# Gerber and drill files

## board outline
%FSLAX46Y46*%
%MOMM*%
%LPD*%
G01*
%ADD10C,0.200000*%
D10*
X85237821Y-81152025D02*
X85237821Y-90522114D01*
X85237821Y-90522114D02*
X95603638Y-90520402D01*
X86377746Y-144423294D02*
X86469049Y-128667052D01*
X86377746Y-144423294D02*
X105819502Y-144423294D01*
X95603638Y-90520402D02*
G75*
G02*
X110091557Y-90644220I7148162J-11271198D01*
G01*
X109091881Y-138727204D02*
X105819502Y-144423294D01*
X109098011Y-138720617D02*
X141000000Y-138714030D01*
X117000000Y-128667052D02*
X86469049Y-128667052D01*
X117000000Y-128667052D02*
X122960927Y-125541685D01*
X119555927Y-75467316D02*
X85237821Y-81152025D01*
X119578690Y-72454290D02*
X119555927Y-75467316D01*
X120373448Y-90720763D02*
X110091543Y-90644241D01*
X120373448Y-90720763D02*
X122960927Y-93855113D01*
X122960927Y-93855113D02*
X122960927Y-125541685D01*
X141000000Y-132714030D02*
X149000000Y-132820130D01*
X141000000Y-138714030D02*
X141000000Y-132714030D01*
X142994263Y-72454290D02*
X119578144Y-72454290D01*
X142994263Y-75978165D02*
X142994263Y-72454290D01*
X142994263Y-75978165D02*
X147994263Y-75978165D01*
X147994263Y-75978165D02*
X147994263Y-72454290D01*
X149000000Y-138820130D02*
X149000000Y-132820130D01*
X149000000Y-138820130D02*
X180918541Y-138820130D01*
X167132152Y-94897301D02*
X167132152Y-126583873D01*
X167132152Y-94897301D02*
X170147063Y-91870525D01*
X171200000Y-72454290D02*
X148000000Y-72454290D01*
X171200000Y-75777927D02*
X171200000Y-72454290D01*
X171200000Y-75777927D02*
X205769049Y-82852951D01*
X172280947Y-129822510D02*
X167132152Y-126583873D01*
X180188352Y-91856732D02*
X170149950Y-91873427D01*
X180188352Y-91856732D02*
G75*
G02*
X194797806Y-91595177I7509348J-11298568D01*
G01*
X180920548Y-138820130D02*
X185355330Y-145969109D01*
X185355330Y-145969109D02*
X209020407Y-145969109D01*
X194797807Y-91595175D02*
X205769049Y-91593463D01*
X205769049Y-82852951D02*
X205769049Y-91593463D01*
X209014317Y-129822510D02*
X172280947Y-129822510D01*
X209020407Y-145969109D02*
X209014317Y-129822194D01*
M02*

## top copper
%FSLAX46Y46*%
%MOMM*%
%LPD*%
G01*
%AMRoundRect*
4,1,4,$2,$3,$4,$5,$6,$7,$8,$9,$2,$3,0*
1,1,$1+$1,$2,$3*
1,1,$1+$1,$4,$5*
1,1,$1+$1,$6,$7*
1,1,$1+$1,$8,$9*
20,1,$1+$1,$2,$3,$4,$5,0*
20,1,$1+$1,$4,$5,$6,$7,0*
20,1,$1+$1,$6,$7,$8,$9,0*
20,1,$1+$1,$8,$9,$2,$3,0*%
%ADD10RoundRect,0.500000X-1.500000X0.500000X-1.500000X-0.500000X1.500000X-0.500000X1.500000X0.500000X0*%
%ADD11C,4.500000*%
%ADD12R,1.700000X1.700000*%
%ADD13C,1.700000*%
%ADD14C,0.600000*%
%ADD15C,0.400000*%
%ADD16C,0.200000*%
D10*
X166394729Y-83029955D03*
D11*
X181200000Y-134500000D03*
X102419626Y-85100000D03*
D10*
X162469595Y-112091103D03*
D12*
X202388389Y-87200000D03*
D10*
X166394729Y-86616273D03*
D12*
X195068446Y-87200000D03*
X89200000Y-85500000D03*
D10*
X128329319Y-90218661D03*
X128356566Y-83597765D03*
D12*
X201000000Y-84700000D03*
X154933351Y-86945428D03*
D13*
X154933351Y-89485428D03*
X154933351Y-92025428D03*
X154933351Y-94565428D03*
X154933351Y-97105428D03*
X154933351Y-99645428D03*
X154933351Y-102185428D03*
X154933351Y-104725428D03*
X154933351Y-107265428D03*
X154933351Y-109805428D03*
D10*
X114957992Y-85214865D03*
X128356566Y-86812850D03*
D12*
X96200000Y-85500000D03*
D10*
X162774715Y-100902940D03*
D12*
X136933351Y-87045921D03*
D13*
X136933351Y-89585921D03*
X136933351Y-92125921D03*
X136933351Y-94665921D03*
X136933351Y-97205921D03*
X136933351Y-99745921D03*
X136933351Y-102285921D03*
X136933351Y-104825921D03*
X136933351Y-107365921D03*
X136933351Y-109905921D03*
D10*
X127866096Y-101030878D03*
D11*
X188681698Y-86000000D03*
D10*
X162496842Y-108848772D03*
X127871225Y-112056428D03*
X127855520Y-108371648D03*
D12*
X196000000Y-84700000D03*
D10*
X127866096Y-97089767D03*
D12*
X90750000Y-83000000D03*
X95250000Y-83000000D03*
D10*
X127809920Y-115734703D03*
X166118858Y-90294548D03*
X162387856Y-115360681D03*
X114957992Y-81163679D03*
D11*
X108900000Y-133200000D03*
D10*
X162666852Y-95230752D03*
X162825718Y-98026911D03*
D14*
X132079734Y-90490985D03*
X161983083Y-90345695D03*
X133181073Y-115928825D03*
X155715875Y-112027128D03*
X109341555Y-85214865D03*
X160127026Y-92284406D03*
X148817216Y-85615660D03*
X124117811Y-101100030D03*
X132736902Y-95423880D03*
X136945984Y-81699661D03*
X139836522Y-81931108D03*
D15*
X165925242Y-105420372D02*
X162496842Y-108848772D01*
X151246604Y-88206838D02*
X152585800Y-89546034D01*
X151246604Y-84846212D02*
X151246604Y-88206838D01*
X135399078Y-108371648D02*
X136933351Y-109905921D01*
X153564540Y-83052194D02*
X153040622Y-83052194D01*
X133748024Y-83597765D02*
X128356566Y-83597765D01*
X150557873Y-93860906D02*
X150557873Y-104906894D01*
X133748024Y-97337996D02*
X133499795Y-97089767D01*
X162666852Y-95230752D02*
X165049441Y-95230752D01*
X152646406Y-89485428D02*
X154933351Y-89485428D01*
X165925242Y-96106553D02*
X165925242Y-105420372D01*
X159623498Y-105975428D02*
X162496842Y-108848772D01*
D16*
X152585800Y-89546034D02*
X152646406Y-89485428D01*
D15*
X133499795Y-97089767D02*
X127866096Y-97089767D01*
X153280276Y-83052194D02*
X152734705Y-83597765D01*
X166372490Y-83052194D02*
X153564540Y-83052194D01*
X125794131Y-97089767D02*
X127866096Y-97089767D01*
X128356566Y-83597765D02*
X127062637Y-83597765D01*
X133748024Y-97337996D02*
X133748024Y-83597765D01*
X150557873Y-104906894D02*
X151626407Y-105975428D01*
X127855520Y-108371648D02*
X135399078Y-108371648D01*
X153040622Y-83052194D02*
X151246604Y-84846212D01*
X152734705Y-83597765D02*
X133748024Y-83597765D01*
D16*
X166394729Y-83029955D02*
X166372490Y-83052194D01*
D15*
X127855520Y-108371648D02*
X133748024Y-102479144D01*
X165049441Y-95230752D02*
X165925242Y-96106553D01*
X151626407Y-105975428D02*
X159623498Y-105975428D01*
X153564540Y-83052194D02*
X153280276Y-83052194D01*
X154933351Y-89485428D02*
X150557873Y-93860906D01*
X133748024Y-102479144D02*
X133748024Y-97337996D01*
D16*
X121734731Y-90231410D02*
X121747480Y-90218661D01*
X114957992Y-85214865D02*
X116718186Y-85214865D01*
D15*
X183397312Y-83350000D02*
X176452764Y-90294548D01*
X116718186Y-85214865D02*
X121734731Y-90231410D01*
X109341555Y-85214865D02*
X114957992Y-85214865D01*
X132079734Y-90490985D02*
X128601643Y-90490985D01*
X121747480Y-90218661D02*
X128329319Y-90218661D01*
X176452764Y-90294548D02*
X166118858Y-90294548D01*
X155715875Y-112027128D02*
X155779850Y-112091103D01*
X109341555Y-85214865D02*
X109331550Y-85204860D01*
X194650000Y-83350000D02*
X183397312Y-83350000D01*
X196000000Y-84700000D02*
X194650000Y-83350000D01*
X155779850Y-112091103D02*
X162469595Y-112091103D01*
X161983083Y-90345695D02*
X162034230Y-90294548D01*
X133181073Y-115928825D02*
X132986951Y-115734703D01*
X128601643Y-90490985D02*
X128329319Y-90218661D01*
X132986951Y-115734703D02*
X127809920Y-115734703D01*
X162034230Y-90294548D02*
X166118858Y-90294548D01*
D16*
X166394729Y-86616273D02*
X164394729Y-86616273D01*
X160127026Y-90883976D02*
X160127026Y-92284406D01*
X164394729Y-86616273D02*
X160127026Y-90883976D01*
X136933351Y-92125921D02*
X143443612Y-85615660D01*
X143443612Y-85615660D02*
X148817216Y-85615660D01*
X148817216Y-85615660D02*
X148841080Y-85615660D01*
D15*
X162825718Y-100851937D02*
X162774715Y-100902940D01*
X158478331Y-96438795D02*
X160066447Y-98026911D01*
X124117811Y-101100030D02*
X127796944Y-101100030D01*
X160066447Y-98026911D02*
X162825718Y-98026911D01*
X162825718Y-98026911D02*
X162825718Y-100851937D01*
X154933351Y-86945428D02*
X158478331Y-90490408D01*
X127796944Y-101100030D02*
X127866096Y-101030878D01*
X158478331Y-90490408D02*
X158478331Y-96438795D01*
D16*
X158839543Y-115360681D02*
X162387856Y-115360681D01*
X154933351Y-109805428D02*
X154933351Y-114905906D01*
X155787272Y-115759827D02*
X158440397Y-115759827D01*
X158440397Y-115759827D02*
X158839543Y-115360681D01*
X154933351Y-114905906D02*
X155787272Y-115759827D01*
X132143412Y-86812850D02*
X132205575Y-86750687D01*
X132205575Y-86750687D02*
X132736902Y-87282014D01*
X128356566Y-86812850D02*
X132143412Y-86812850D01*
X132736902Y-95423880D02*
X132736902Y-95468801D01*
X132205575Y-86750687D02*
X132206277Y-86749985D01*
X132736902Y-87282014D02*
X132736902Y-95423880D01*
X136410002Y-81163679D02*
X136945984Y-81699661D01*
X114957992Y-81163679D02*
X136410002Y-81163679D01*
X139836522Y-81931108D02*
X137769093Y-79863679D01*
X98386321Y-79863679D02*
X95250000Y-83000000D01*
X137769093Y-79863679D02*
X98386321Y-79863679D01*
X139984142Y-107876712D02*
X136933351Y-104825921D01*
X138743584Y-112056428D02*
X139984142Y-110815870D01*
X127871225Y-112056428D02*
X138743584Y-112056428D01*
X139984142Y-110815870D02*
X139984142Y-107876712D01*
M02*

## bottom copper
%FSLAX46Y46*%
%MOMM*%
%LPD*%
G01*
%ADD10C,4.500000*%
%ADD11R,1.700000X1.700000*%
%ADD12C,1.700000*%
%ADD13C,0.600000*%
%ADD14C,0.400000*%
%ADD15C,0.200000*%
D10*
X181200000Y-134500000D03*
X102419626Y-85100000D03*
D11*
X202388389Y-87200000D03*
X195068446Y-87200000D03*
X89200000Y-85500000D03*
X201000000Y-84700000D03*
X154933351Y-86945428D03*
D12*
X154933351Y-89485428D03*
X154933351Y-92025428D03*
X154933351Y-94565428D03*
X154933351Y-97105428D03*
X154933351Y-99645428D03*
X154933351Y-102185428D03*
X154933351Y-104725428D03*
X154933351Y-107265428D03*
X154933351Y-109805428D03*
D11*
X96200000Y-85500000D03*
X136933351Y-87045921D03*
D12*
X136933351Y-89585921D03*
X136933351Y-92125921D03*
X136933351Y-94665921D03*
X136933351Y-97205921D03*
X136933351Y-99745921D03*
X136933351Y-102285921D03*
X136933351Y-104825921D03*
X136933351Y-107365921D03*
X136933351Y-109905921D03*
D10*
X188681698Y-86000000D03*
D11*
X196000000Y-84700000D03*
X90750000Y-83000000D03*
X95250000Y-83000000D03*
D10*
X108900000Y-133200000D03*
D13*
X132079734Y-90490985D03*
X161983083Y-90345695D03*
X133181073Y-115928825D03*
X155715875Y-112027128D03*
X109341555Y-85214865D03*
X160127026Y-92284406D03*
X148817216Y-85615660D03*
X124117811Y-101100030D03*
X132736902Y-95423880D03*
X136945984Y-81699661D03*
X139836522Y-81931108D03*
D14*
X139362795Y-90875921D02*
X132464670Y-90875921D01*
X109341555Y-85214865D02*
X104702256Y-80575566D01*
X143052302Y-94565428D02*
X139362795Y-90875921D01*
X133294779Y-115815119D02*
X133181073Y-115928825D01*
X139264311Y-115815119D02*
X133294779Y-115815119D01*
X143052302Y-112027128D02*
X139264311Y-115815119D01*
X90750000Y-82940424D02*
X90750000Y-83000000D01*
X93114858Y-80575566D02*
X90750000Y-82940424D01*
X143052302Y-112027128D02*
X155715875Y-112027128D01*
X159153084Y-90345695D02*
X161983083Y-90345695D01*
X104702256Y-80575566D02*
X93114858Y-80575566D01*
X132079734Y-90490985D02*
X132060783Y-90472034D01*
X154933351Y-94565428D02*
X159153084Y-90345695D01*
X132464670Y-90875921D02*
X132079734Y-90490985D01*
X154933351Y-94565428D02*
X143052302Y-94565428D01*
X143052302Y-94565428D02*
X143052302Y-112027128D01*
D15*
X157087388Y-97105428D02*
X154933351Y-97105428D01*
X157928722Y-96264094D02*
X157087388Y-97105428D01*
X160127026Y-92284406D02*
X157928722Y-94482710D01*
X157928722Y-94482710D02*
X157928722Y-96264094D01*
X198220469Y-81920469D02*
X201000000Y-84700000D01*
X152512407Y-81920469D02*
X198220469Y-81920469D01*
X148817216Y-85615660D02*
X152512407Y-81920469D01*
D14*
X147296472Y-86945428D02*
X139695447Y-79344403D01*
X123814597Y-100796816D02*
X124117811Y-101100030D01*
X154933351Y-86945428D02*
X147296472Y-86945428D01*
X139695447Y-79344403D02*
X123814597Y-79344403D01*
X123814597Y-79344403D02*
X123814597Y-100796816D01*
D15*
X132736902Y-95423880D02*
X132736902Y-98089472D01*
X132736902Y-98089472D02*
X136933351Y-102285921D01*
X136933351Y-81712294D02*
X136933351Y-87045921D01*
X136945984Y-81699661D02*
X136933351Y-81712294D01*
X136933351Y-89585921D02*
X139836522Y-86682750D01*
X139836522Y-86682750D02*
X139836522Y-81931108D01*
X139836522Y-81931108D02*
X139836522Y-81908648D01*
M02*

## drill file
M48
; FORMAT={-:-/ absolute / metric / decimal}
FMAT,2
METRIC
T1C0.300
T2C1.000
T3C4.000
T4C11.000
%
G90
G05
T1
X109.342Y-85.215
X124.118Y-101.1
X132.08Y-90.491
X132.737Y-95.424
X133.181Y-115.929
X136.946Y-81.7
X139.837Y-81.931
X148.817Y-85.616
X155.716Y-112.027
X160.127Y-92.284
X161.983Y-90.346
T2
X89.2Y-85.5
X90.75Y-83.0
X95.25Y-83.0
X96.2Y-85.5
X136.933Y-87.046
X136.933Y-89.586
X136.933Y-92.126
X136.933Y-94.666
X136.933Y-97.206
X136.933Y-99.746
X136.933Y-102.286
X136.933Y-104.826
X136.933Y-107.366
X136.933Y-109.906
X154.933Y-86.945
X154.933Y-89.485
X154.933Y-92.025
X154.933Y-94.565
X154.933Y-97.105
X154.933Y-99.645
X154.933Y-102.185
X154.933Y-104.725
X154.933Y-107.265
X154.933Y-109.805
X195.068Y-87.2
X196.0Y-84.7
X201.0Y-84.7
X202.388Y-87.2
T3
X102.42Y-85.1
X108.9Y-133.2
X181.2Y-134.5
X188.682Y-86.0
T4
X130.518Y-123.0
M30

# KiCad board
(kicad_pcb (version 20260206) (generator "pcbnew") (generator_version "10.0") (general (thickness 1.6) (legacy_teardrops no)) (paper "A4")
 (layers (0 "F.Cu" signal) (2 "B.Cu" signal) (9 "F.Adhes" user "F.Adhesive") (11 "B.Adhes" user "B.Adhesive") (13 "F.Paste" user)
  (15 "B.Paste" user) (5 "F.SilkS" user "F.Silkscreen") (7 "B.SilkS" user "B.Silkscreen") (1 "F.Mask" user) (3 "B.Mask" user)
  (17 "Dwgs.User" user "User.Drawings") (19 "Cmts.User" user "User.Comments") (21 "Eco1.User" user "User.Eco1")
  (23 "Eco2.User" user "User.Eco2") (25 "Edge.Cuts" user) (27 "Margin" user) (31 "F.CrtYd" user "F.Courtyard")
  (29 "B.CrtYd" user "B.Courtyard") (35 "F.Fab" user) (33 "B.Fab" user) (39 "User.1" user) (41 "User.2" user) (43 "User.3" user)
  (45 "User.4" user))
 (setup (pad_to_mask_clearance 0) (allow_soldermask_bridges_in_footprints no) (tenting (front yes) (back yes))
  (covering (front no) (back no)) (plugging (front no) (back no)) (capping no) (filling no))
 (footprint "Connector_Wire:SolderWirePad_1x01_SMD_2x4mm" (layer "F.Cu") (at 166.394729 83.029955 -90)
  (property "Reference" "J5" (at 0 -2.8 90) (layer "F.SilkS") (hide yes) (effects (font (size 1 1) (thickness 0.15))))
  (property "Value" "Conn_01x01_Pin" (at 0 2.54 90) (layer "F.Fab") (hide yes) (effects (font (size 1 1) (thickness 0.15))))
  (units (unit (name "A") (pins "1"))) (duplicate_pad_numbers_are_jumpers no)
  (pad "1" smd roundrect (at 0 0 270) (size 2 4) (layers "F.Cu" "F.Mask") (roundrect_rratio 0.25) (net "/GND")))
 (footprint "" (layer "F.Cu") (at 199.537516 63.787243)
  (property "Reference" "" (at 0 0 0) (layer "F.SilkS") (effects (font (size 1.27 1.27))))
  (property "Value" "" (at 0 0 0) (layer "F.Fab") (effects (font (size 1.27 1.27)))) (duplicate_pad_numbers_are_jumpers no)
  (pad "" np_thru_hole circle (at -18.337516 70.712757) (size 4.5 4.5) (drill 4) (layers "*.Cu" "*.Mask")))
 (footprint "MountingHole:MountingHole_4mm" (layer "F.Cu") (at 102.419626 85.1)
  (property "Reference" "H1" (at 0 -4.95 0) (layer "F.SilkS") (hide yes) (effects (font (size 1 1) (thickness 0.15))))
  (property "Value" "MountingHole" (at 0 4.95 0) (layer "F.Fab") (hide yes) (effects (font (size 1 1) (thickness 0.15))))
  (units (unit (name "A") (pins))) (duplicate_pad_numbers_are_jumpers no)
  (pad "" np_thru_hole circle (at 0 0) (size 4.5 4.5) (drill 4) (layers "*.Cu" "*.Mask")))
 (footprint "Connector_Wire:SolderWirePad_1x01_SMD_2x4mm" (layer "F.Cu") (at 162.469595 112.091103 -90)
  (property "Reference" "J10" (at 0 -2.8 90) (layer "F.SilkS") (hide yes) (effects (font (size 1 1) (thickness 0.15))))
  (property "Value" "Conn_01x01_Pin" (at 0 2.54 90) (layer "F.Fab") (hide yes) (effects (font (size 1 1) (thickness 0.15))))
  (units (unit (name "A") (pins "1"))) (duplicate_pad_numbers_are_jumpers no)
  (pad "1" smd roundrect (at 0 0 270) (size 2 4) (layers "F.Cu" "F.Mask") (roundrect_rratio 0.25) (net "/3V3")))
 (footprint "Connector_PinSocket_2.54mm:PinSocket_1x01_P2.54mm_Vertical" (layer "F.Cu") (at 202.388389 87.2)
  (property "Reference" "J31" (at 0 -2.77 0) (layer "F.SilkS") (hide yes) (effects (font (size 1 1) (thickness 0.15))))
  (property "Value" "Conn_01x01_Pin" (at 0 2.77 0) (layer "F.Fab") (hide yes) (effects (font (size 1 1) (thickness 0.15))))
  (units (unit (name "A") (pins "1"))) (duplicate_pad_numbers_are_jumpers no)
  (pad "1" thru_hole rect (at 0 0) (size 1.7 1.7) (drill 1) (layers "*.Cu" "*.Mask") (remove_unused_layers no)
   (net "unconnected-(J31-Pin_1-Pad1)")))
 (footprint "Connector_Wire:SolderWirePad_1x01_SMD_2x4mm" (layer "F.Cu") (at 166.394729 86.616273 -90)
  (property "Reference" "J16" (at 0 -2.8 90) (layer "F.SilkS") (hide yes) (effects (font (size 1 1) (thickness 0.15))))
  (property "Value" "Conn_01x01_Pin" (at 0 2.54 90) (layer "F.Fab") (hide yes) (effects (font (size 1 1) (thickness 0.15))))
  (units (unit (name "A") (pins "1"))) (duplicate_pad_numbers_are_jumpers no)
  (pad "1" smd roundrect (at 0 0 270) (size 2 4) (layers "F.Cu" "F.Mask") (roundrect_rratio 0.25) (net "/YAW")))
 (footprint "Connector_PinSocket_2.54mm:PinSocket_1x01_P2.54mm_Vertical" (layer "F.Cu") (at 195.068446 87.2)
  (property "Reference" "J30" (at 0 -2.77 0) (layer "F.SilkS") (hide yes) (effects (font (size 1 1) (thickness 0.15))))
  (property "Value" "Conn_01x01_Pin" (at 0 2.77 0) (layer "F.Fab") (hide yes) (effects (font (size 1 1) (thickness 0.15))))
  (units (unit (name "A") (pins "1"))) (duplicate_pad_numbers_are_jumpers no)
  (pad "1" thru_hole rect (at 0 0) (size 1.7 1.7) (drill 1) (layers "*.Cu" "*.Mask") (remove_unused_layers no)
   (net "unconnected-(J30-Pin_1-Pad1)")))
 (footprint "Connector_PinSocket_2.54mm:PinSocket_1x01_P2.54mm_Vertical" (layer "F.Cu") (at 89.2 85.5)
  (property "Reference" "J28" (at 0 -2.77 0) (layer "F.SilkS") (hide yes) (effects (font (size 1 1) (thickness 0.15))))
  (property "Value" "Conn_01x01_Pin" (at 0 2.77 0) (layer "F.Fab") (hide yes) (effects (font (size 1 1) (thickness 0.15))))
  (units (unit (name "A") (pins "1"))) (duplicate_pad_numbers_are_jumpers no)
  (pad "1" thru_hole rect (at 0 0) (size 1.7 1.7) (drill 1) (layers "*.Cu" "*.Mask") (remove_unused_layers no)
   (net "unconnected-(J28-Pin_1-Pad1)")))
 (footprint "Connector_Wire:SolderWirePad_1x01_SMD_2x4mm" (layer "F.Cu") (at 128.329319 90.218661 -90)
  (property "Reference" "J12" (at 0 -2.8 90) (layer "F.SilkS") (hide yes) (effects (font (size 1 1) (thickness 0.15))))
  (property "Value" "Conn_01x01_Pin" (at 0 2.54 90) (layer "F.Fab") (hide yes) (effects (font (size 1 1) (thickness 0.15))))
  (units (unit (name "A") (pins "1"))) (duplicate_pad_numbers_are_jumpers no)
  (pad "1" smd roundrect (at 0 0 270) (size 2 4) (layers "F.Cu" "F.Mask") (roundrect_rratio 0.25) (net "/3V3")))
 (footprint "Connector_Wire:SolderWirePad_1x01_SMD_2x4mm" (layer "F.Cu") (at 128.356566 83.597765 -90)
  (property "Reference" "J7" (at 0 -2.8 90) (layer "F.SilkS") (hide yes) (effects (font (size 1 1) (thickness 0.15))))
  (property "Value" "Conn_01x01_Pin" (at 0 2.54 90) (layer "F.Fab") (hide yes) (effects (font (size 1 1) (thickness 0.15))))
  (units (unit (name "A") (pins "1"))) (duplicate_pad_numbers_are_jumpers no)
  (pad "1" smd roundrect (at 0 0 270) (size 2 4) (layers "F.Cu" "F.Mask") (roundrect_rratio 0.25) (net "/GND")))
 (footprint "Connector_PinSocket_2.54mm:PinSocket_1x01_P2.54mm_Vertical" (layer "F.Cu") (at 201 84.7)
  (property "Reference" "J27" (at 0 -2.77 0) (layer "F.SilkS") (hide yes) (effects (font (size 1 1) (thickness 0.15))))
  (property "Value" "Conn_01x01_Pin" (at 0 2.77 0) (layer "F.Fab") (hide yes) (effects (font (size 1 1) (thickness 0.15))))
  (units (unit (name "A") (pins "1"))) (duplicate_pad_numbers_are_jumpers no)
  (pad "1" thru_hole rect (at 0 0) (size 1.7 1.7) (drill 1) (layers "*.Cu" "*.Mask") (remove_unused_layers no) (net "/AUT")))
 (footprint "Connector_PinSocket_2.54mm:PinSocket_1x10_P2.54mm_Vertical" (layer "F.Cu") (at 154.933351 86.945428)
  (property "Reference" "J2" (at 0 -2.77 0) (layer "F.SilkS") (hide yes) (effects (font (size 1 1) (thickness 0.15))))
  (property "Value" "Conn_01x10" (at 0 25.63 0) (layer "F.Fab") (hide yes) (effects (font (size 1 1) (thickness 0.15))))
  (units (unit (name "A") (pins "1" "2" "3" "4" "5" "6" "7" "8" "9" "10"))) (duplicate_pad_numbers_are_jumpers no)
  (pad "1" thru_hole rect (at 0 0) (size 1.7 1.7) (drill 1) (layers "*.Cu" "*.Mask") (remove_unused_layers no) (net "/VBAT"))
  (pad "2" thru_hole circle (at 0 2.54) (size 1.7 1.7) (drill 1) (layers "*.Cu" "*.Mask") (remove_unused_layers no) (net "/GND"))
  (pad "3" thru_hole circle (at 0 5.08) (size 1.7 1.7) (drill 1) (layers "*.Cu" "*.Mask") (remove_unused_layers no) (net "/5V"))
  (pad "4" thru_hole circle (at 0 7.62) (size 1.7 1.7) (drill 1) (layers "*.Cu" "*.Mask") (remove_unused_layers no) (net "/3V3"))
  (pad "5" thru_hole circle (at 0 10.16) (size 1.7 1.7) (drill 1) (layers "*.Cu" "*.Mask") (remove_unused_layers no) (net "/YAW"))
  (pad "6" thru_hole circle (at 0 12.7) (size 1.7 1.7) (drill 1) (layers "*.Cu" "*.Mask") (remove_unused_layers no)
   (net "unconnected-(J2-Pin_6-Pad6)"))
  (pad "7" thru_hole circle (at 0 15.24) (size 1.7 1.7) (drill 1) (layers "*.Cu" "*.Mask") (remove_unused_layers no)
   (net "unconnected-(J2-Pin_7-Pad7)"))
  (pad "8" thru_hole circle (at 0 17.78) (size 1.7 1.7) (drill 1) (layers "*.Cu" "*.Mask") (remove_unused_layers no)
   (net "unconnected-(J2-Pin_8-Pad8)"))
  (pad "9" thru_hole circle (at 0 20.32) (size 1.7 1.7) (drill 1) (layers "*.Cu" "*.Mask") (remove_unused_layers no)
   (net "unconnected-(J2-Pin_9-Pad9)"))
  (pad "10" thru_hole circle (at 0 22.86) (size 1.7 1.7) (drill 1) (layers "*.Cu" "*.Mask") (remove_unused_layers no) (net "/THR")))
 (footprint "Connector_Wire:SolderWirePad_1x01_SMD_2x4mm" (layer "F.Cu") (at 114.957992 85.214865 -90)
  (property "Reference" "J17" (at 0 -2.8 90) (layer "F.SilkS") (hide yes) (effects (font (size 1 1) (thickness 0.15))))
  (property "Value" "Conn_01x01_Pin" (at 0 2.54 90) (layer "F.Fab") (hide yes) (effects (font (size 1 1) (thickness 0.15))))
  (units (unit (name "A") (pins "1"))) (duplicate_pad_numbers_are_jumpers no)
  (pad "1" smd roundrect (at 0 0 270) (size 2 4) (layers "F.Cu" "F.Mask") (roundrect_rratio 0.25) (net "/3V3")))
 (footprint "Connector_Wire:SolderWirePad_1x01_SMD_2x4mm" (layer "F.Cu") (at 128.356566 86.81285 -90)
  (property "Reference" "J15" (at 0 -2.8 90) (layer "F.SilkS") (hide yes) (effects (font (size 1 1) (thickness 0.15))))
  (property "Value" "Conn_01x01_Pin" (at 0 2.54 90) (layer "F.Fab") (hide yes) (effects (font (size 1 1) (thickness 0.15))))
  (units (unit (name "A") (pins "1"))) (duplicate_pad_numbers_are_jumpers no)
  (pad "1" smd roundrect (at 0 0 270) (size 2 4) (layers "F.Cu" "F.Mask") (roundrect_rratio 0.25) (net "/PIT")))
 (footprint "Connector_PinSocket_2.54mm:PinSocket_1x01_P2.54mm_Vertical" (layer "F.Cu") (at 96.2 85.5)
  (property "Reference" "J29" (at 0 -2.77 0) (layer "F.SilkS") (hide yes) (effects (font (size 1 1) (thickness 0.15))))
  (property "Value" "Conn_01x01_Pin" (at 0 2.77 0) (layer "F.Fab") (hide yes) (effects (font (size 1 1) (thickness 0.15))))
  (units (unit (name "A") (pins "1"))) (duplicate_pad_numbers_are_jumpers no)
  (pad "1" thru_hole rect (at 0 0) (size 1.7 1.7) (drill 1) (layers "*.Cu" "*.Mask") (remove_unused_layers no)
   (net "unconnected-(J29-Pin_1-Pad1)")))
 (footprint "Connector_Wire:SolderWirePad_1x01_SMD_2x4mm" (layer "F.Cu") (at 162.774715 100.90294 -90)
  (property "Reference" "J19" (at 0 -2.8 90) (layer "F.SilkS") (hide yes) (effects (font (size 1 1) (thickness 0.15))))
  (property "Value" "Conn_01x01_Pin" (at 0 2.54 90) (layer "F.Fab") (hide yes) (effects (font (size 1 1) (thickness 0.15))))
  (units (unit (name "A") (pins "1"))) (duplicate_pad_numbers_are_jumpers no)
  (pad "1" smd roundrect (at 0 0 270) (size 2 4) (layers "F.Cu" "F.Mask") (roundrect_rratio 0.25) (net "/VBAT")))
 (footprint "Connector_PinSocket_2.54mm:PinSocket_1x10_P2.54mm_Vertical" (layer "F.Cu") (at 136.933351 87.045921)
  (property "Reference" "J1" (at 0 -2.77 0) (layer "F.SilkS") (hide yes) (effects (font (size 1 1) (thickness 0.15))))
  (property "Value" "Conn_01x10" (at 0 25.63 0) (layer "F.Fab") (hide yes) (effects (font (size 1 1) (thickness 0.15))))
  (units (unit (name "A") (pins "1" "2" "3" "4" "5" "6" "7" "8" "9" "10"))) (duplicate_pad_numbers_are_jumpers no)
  (pad "1" thru_hole rect (at 0 0) (size 1.7 1.7) (drill 1) (layers "*.Cu" "*.Mask") (remove_unused_layers no) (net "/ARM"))
  (pad "2" thru_hole circle (at 0 2.54) (size 1.7 1.7) (drill 1) (layers "*.Cu" "*.Mask") (remove_unused_layers no) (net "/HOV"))
  (pad "3" thru_hole circle (at 0 5.08) (size 1.7 1.7) (drill 1) (layers "*.Cu" "*.Mask") (remove_unused_layers no) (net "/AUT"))
  (pad "4" thru_hole circle (at 0 7.62) (size 1.7 1.7) (drill 1) (layers "*.Cu" "*.Mask") (remove_unused_layers no) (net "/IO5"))
  (pad "5" thru_hole circle (at 0 10.16) (size 1.7 1.7) (drill 1) (layers "*.Cu" "*.Mask") (remove_unused_layers no) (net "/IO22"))
  (pad "6" thru_hole circle (at 0 12.7) (size 1.7 1.7) (drill 1) (layers "*.Cu" "*.Mask") (remove_unused_layers no) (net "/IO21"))
  (pad "7" thru_hole circle (at 0 15.24) (size 1.7 1.7) (drill 1) (layers "*.Cu" "*.Mask") (remove_unused_layers no) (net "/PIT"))
  (pad "8" thru_hole circle (at 0 17.78) (size 1.7 1.7) (drill 1) (layers "*.Cu" "*.Mask") (remove_unused_layers no) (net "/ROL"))
  (pad "9" thru_hole circle (at 0 20.32) (size 1.7 1.7) (drill 1) (layers "*.Cu" "*.Mask") (remove_unused_layers no) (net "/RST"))
  (pad "10" thru_hole circle (at 0 22.86) (size 1.7 1.7) (drill 1) (layers "*.Cu" "*.Mask") (remove_unused_layers no) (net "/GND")))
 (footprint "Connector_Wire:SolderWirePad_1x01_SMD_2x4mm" (layer "F.Cu") (at 127.866096 101.030878 -90)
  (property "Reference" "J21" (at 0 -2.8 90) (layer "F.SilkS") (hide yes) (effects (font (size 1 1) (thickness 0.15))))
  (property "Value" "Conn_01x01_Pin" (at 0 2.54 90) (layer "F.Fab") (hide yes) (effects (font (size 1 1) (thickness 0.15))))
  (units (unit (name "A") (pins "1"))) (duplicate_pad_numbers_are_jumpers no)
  (pad "1" smd roundrect (at 0 0 270) (size 2 4) (layers "F.Cu" "F.Mask") (roundrect_rratio 0.25) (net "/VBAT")))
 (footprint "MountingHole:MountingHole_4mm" (layer "F.Cu") (at 188.681698 86)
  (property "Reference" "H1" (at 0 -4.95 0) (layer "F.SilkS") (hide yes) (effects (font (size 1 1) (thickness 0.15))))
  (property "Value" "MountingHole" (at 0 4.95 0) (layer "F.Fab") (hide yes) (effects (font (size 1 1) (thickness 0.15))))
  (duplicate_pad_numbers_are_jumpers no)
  (pad "" np_thru_hole circle (at 0 0) (size 4.5 4.5) (drill 4) (layers "*.Cu" "*.Mask")))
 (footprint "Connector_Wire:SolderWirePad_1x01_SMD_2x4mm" (layer "F.Cu") (at 162.496842 108.848772 -90)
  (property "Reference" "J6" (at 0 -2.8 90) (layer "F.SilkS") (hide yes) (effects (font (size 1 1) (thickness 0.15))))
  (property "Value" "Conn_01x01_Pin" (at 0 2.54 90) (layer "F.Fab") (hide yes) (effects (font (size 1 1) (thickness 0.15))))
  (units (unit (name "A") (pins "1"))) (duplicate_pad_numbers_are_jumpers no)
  (pad "1" smd roundrect (at 0 0 270) (size 2 4) (layers "F.Cu" "F.Mask") (roundrect_rratio 0.25) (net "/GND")))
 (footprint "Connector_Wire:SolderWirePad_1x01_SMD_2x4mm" (layer "F.Cu") (at 127.871225 112.056428 -90)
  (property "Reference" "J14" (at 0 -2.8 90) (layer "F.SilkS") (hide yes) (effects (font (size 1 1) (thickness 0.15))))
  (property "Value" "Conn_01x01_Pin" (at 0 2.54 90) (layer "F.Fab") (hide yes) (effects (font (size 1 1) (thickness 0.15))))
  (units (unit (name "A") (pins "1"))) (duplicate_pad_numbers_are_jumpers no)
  (pad "1" smd roundrect (at 0 0 270) (size 2 4) (layers "F.Cu" "F.Mask") (roundrect_rratio 0.25) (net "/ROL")))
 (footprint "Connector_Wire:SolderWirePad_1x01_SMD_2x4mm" (layer "F.Cu") (at 127.85552 108.371648 -90)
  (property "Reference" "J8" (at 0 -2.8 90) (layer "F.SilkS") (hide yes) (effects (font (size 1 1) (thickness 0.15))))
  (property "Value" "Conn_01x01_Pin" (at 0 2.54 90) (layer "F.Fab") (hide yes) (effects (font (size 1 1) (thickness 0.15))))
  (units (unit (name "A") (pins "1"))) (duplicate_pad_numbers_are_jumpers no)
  (pad "1" smd roundrect (at 0 0 270) (size 2 4) (layers "F.Cu" "F.Mask") (roundrect_rratio 0.25) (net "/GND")))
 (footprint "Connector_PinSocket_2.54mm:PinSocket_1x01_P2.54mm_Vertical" (layer "F.Cu") (at 196 84.7)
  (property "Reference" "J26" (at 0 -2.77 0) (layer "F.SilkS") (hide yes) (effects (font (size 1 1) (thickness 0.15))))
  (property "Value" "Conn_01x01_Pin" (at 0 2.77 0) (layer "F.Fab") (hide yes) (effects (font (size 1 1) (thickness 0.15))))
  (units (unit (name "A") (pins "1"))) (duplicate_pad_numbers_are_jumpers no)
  (pad "1" thru_hole rect (at 0 0) (size 1.7 1.7) (drill 1) (layers "*.Cu" "*.Mask") (remove_unused_layers no) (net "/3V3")))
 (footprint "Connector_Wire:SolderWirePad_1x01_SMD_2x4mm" (layer "F.Cu") (at 127.866096 97.089767 -90)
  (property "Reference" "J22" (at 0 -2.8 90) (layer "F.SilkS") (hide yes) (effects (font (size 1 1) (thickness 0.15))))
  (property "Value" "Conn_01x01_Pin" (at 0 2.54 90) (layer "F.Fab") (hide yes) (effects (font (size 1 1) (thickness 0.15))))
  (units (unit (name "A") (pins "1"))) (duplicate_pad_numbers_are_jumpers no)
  (pad "1" smd roundrect (at 0 0 270) (size 2 4) (layers "F.Cu" "F.Mask") (roundrect_rratio 0.25) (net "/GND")))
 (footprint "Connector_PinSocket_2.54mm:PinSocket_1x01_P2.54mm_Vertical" (layer "F.Cu") (at 90.75 83)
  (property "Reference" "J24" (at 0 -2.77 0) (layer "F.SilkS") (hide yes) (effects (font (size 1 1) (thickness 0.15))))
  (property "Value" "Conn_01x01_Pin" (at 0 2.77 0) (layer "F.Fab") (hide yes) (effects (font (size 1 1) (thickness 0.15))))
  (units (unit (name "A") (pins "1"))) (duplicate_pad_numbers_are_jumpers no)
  (pad "1" thru_hole rect (at 0 0) (size 1.7 1.7) (drill 1) (layers "*.Cu" "*.Mask") (remove_unused_layers no) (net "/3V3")))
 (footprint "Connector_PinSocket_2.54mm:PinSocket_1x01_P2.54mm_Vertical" (layer "F.Cu") (at 95.25 83)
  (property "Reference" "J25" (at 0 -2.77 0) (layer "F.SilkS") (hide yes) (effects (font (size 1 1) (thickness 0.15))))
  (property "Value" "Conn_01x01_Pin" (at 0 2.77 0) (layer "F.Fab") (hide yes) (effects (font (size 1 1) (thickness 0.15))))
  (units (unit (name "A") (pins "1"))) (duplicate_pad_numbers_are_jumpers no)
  (pad "1" thru_hole rect (at 0 0) (size 1.7 1.7) (drill 1) (layers "*.Cu" "*.Mask") (remove_unused_layers no) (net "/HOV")))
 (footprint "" (layer "F.Cu") (at 131 123 180)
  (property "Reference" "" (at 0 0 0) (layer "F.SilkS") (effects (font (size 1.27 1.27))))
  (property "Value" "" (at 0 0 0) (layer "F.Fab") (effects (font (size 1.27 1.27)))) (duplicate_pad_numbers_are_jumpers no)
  (pad "" np_thru_hole circle (at 0.482324 0 180) (size 11 11) (drill 11) (layers "*.Cu" "*.Mask")))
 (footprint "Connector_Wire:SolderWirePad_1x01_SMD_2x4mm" (layer "F.Cu") (at 127.80992 115.734703 -90)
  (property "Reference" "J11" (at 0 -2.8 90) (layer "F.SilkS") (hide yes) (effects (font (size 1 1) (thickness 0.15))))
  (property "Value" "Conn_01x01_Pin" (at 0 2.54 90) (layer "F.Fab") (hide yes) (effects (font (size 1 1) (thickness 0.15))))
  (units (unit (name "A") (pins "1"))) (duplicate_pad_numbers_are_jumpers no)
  (pad "1" smd roundrect (at 0 0 270) (size 2 4) (layers "F.Cu" "F.Mask") (roundrect_rratio 0.25) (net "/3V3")))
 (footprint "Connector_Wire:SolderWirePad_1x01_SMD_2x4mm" (layer "F.Cu") (at 166.118858 90.294548 -90)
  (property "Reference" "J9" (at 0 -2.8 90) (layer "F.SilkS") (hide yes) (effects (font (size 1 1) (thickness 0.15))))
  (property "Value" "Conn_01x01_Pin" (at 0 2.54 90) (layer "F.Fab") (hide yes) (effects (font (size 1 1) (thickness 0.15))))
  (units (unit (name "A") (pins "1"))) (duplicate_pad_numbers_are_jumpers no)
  (pad "1" smd roundrect (at 0 0 270) (size 2 4) (layers "F.Cu" "F.Mask") (roundrect_rratio 0.25) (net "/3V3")))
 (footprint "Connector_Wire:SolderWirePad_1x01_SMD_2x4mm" (layer "F.Cu") (at 162.387856 115.360681 -90)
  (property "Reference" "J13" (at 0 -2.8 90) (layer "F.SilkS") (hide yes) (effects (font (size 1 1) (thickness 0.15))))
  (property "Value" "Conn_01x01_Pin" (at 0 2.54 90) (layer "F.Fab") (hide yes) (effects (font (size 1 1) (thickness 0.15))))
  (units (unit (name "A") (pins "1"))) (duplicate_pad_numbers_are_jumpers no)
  (pad "1" smd roundrect (at 0 0 270) (size 2 4) (layers "F.Cu" "F.Mask") (roundrect_rratio 0.25) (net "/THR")))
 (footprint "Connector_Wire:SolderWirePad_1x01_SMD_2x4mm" (layer "F.Cu") (at 114.957992 81.163679 -90)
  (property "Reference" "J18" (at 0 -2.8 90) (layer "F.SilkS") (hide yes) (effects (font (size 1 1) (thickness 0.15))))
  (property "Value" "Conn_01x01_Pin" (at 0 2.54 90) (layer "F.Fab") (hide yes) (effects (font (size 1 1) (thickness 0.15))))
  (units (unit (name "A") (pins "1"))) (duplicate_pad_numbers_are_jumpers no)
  (pad "1" smd roundrect (at 0 0 270) (size 2 4) (layers "F.Cu" "F.Mask") (roundrect_rratio 0.25) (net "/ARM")))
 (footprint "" (layer "F.Cu") (at 98.892008 62.425329)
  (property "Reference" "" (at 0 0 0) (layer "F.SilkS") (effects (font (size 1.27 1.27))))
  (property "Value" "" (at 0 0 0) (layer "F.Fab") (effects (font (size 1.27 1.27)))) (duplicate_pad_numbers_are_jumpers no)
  (pad "" np_thru_hole circle (at 10.007992 70.774671) (size 4.5 4.5) (drill 4) (layers "*.Cu" "*.Mask")))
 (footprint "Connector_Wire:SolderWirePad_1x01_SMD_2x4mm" (layer "F.Cu") (at 162.666852 95.230752 -90)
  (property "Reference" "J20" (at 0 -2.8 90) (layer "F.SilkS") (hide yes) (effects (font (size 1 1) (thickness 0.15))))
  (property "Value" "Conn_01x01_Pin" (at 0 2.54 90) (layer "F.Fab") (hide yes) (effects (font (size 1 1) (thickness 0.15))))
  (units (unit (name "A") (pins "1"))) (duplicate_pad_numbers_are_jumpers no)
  (pad "1" smd roundrect (at 0 0 270) (size 2 4) (layers "F.Cu" "F.Mask") (roundrect_rratio 0.25) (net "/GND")))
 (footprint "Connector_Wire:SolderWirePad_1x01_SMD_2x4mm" (layer "F.Cu") (at 162.825718 98.026911 -90)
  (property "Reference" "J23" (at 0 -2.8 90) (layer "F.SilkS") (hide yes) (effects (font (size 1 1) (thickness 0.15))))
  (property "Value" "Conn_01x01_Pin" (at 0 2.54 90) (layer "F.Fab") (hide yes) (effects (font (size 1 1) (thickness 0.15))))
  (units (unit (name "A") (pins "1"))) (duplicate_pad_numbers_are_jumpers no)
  (pad "1" smd roundrect (at 0 0 270) (size 2 4) (layers "F.Cu" "F.Mask") (roundrect_rratio 0.25) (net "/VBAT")))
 (gr_line (start 85.237821 81.152025) (end 85.237821 90.522114) (stroke (width 0.2) (type solid)) (layer "Edge.Cuts"))
 (gr_line (start 85.237821 90.522114) (end 95.603638 90.520402) (stroke (width 0.2) (type solid)) (layer "Edge.Cuts"))
 (gr_line (start 86.377746 144.423294) (end 86.469049 128.667052) (stroke (width 0.2) (type solid)) (layer "Edge.Cuts"))
 (gr_line (start 86.377746 144.423294) (end 105.819502 144.423294) (stroke (width 0.2) (type solid)) (layer "Edge.Cuts"))
 (gr_arc (start 95.603638 90.520402) (mid 102.865857 88.445339) (end 110.091543 90.644241) (stroke (width 0.2) (type solid))
  (layer "Edge.Cuts"))
 (gr_line (start 109.091881 138.727204) (end 105.819502 144.423294) (stroke (width 0.2) (type solid)) (layer "Edge.Cuts"))
 (gr_line (start 109.098011 138.720617) (end 141 138.71403) (stroke (width 0.2) (type solid)) (layer "Edge.Cuts"))
 (gr_line (start 117 128.667052) (end 86.469049 128.667052) (stroke (width 0.2) (type solid)) (layer "Edge.Cuts"))
 (gr_line (start 117 128.667052) (end 122.960927 125.541685) (stroke (width 0.2) (type solid)) (layer "Edge.Cuts"))
 (gr_line (start 119.555927 75.467316) (end 85.237821 81.152025) (stroke (width 0.2) (type solid)) (layer "Edge.Cuts"))
 (gr_line (start 119.57869 72.45429) (end 119.555927 75.467316) (stroke (width 0.2) (type solid)) (layer "Edge.Cuts"))
 (gr_line (start 120.373448 90.720763) (end 110.091543 90.644241) (stroke (width 0.2) (type solid)) (layer "Edge.Cuts"))
 (gr_line (start 120.373448 90.720763) (end 122.960927 93.855113) (stroke (width 0.2) (type solid)) (layer "Edge.Cuts"))
 (gr_line (start 122.960927 93.855113) (end 122.960927 125.541685) (stroke (width 0.2) (type solid)) (layer "Edge.Cuts"))
 (gr_line (start 141 132.71403) (end 149 132.82013) (stroke (width 0.2) (type solid)) (layer "Edge.Cuts"))
 (gr_line (start 141 138.71403) (end 141 132.71403) (stroke (width 0.2) (type solid)) (layer "Edge.Cuts"))
 (gr_line (start 142.994263 72.45429) (end 119.578144 72.45429) (stroke (width 0.2) (type solid)) (layer "Edge.Cuts"))
 (gr_line (start 142.994263 75.978165) (end 142.994263 72.45429) (stroke (width 0.2) (type solid)) (layer "Edge.Cuts"))
 (gr_line (start 142.994263 75.978165) (end 147.994263 75.978165) (stroke (width 0.2) (type solid)) (layer "Edge.Cuts"))
 (gr_line (start 147.994263 75.978165) (end 147.994263 72.45429) (stroke (width 0.2) (type solid)) (layer "Edge.Cuts"))
 (gr_line (start 149 138.82013) (end 149 132.82013) (stroke (width 0.2) (type solid)) (layer "Edge.Cuts"))
 (gr_line (start 149 138.82013) (end 180.918541 138.82013) (stroke (width 0.2) (type solid)) (layer "Edge.Cuts"))
 (gr_line (start 167.132152 94.897301) (end 167.132152 126.583873) (stroke (width 0.2) (type solid)) (layer "Edge.Cuts"))
 (gr_line (start 167.132152 94.897301) (end 170.147063 91.870525) (stroke (width 0.2) (type solid)) (layer "Edge.Cuts"))
 (gr_line (start 171.2 72.45429) (end 148 72.45429) (stroke (width 0.2) (type solid)) (layer "Edge.Cuts"))
 (gr_line (start 171.2 75.777927) (end 171.2 72.45429) (stroke (width 0.2) (type solid)) (layer "Edge.Cuts"))
 (gr_line (start 171.2 75.777927) (end 205.769049 82.852951) (stroke (width 0.2) (type solid)) (layer "Edge.Cuts"))
 (gr_line (start 172.280947 129.82251) (end 167.132152 126.583873) (stroke (width 0.2) (type solid)) (layer "Edge.Cuts"))
 (gr_line (start 180.188352 91.856732) (end 170.14995 91.873427) (stroke (width 0.2) (type solid)) (layer "Edge.Cuts"))
 (gr_arc (start 180.188352 91.856732) (mid 187.454858 89.591048) (end 194.797807 91.595176) (stroke (width 0.2) (type solid))
  (layer "Edge.Cuts"))
 (gr_line (start 180.920548 138.82013) (end 185.35533 145.969109) (stroke (width 0.2) (type solid)) (layer "Edge.Cuts"))
 (gr_line (start 185.35533 145.969109) (end 209.020407 145.969109) (stroke (width 0.2) (type solid)) (layer "Edge.Cuts"))
 (gr_line (start 194.797807 91.595175) (end 205.769049 91.593463) (stroke (width 0.2) (type solid)) (layer "Edge.Cuts"))
 (gr_line (start 205.769049 82.852951) (end 205.769049 91.593463) (stroke (width 0.2) (type solid)) (layer "Edge.Cuts"))
 (gr_line (start 209.014317 129.82251) (end 172.280947 129.82251) (stroke (width 0.2) (type solid)) (layer "Edge.Cuts"))
 (gr_line (start 209.020407 145.969109) (end 209.014317 129.822194) (stroke (width 0.2) (type solid)) (layer "Edge.Cuts"))
 (segment (start 165.925242 105.420372) (end 162.496842 108.848772) (width 0.4) (layer "F.Cu") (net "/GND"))
 (segment (start 151.246604 88.206838) (end 152.5858 89.546034) (width 0.4) (layer "F.Cu") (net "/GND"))
 (segment (start 151.246604 84.846212) (end 151.246604 88.206838) (width 0.4) (layer "F.Cu") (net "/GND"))
 (segment (start 135.399078 108.371648) (end 136.933351 109.905921) (width 0.4) (layer "F.Cu") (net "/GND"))
 (segment (start 153.56454 83.052194) (end 153.040622 83.052194) (width 0.4) (layer "F.Cu") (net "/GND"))
 (segment (start 133.748024 83.597765) (end 128.356566 83.597765) (width 0.4) (layer "F.Cu") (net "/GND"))
 (segment (start 150.557873 93.860906) (end 150.557873 104.906894) (width 0.4) (layer "F.Cu") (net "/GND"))
 (segment (start 133.748024 97.337996) (end 133.499795 97.089767) (width 0.4) (layer "F.Cu") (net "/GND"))
 (segment (start 162.666852 95.230752) (end 165.049441 95.230752) (width 0.4) (layer "F.Cu") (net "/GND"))
 (segment (start 152.646406 89.485428) (end 154.933351 89.485428) (width 0.4) (layer "F.Cu") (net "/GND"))
 (segment (start 165.925242 96.106553) (end 165.925242 105.420372) (width 0.4) (layer "F.Cu") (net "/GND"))
 (segment (start 159.623498 105.975428) (end 162.496842 108.848772) (width 0.4) (layer "F.Cu") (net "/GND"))
 (segment (start 152.5858 89.546034) (end 152.646406 89.485428) (width 0.2) (layer "F.Cu") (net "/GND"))
 (segment (start 133.499795 97.089767) (end 127.866096 97.089767) (width 0.4) (layer "F.Cu") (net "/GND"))
 (segment (start 153.280276 83.052194) (end 152.734705 83.597765) (width 0.4) (layer "F.Cu") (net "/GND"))
 (segment (start 166.37249 83.052194) (end 153.56454 83.052194) (width 0.4) (layer "F.Cu") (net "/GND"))
 (segment (start 125.794131 97.089767) (end 127.866096 97.089767) (width 0.4) (layer "F.Cu") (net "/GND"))
 (segment (start 128.356566 83.597765) (end 127.062637 83.597765) (width 0.4) (layer "F.Cu") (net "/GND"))
 (segment (start 133.748024 97.337996) (end 133.748024 83.597765) (width 0.4) (layer "F.Cu") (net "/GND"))
 (segment (start 150.557873 104.906894) (end 151.626407 105.975428) (width 0.4) (layer "F.Cu") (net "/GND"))
 (segment (start 127.85552 108.371648) (end 135.399078 108.371648) (width 0.4) (layer "F.Cu") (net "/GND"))
 (segment (start 153.040622 83.052194) (end 151.246604 84.846212) (width 0.4) (layer "F.Cu") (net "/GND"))
 (segment (start 152.734705 83.597765) (end 133.748024 83.597765) (width 0.4) (layer "F.Cu") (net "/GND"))
 (segment (start 166.394729 83.029955) (end 166.37249 83.052194) (width 0.2) (layer "F.Cu") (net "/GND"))
 (segment (start 127.85552 108.371648) (end 133.748024 102.479144) (width 0.4) (layer "F.Cu") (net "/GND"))
 (segment (start 165.049441 95.230752) (end 165.925242 96.106553) (width 0.4) (layer "F.Cu") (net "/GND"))
 (segment (start 151.626407 105.975428) (end 159.623498 105.975428) (width 0.4) (layer "F.Cu") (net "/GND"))
 (segment (start 153.56454 83.052194) (end 153.280276 83.052194) (width 0.4) (layer "F.Cu") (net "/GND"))
 (segment (start 154.933351 89.485428) (end 150.557873 93.860906) (width 0.4) (layer "F.Cu") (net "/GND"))
 (segment (start 133.748024 102.479144) (end 133.748024 97.337996) (width 0.4) (layer "F.Cu") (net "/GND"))
 (segment (start 121.734731 90.23141) (end 121.74748 90.218661) (width 0.2) (layer "F.Cu") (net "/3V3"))
 (segment (start 114.957992 85.214865) (end 116.718186 85.214865) (width 0.2) (layer "F.Cu") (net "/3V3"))
 (segment (start 183.397312 83.35) (end 176.452764 90.294548) (width 0.4) (layer "F.Cu") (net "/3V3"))
 (segment (start 116.718186 85.214865) (end 121.734731 90.23141) (width 0.4) (layer "F.Cu") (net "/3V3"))
 (segment (start 109.341555 85.214865) (end 114.957992 85.214865) (width 0.4) (layer "F.Cu") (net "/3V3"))
 (segment (start 132.079734 90.490985) (end 128.601643 90.490985) (width 0.4) (layer "F.Cu") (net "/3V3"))
 (segment (start 121.74748 90.218661) (end 128.329319 90.218661) (width 0.4) (layer "F.Cu") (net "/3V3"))
 (segment (start 176.452764 90.294548) (end 166.118858 90.294548) (width 0.4) (layer "F.Cu") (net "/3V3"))
 (segment (start 155.715875 112.027128) (end 155.77985 112.091103) (width 0.4) (layer "F.Cu") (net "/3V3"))
 (segment (start 109.341555 85.214865) (end 109.33155 85.20486) (width 0.4) (layer "F.Cu") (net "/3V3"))
 (segment (start 194.65 83.35) (end 183.397312 83.35) (width 0.4) (layer "F.Cu") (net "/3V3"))
 (segment (start 196 84.7) (end 194.65 83.35) (width 0.4) (layer "F.Cu") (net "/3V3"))
 (segment (start 155.77985 112.091103) (end 162.469595 112.091103) (width 0.4) (layer "F.Cu") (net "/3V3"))
 (segment (start 161.983083 90.345695) (end 162.03423 90.294548) (width 0.4) (layer "F.Cu") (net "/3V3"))
 (segment (start 133.181073 115.928825) (end 132.986951 115.734703) (width 0.4) (layer "F.Cu") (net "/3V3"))
 (segment (start 128.601643 90.490985) (end 128.329319 90.218661) (width 0.4) (layer "F.Cu") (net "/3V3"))
 (segment (start 132.986951 115.734703) (end 127.80992 115.734703) (width 0.4) (layer "F.Cu") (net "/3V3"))
 (segment (start 162.03423 90.294548) (end 166.118858 90.294548) (width 0.4) (layer "F.Cu") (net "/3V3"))
 (via (at 132.079734 90.490985) (size 0.6) (drill 0.3) (layers "F.Cu" "B.Cu") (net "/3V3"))
 (via (at 161.983083 90.345695) (size 0.6) (drill 0.3) (layers "F.Cu" "B.Cu") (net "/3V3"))
 (via (at 133.181073 115.928825) (size 0.6) (drill 0.3) (layers "F.Cu" "B.Cu") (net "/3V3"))
 (via (at 155.715875 112.027128) (size 0.6) (drill 0.3) (layers "F.Cu" "B.Cu") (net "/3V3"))
 (via (at 109.341555 85.214865) (size 0.6) (drill 0.3) (layers "F.Cu" "B.Cu") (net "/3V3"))
 (segment (start 139.362795 90.875921) (end 132.46467 90.875921) (width 0.4) (layer "B.Cu") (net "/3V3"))
 (segment (start 109.341555 85.214865) (end 104.702256 80.575566) (width 0.4) (layer "B.Cu") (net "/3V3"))
 (segment (start 143.052302 94.565428) (end 139.362795 90.875921) (width 0.4) (layer "B.Cu") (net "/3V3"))
 (segment (start 133.294779 115.815119) (end 133.181073 115.928825) (width 0.4) (layer "B.Cu") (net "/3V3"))
 (segment (start 139.264311 115.815119) (end 133.294779 115.815119) (width 0.4) (layer "B.Cu") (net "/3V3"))
 (segment (start 143.052302 112.027128) (end 139.264311 115.815119) (width 0.4) (layer "B.Cu") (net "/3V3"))
 (segment (start 90.75 82.940424) (end 90.75 83) (width 0.4) (layer "B.Cu") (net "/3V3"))
 (segment (start 93.114858 80.575566) (end 90.75 82.940424) (width 0.4) (layer "B.Cu") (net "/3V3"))
 (segment (start 143.052302 112.027128) (end 155.715875 112.027128) (width 0.4) (layer "B.Cu") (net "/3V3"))
 (segment (start 159.153084 90.345695) (end 161.983083 90.345695) (width 0.4) (layer "B.Cu") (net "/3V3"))
 (segment (start 104.702256 80.575566) (end 93.114858 80.575566) (width 0.4) (layer "B.Cu") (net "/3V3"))
 (segment (start 132.079734 90.490985) (end 132.060783 90.472034) (width 0.4) (layer "B.Cu") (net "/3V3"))
 (segment (start 154.933351 94.565428) (end 159.153084 90.345695) (width 0.4) (layer "B.Cu") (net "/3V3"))
 (segment (start 132.46467 90.875921) (end 132.079734 90.490985) (width 0.4) (layer "B.Cu") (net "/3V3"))
 (segment (start 154.933351 94.565428) (end 143.052302 94.565428) (width 0.4) (layer "B.Cu") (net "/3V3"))
 (segment (start 143.052302 94.565428) (end 143.052302 112.027128) (width 0.4) (layer "B.Cu") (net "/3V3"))
 (segment (start 166.394729 86.616273) (end 164.394729 86.616273) (width 0.2) (layer "F.Cu") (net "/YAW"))
 (segment (start 160.127026 90.883976) (end 160.127026 92.284406) (width 0.2) (layer "F.Cu") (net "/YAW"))
 (segment (start 164.394729 86.616273) (end 160.127026 90.883976) (width 0.2) (layer "F.Cu") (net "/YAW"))
 (via (at 160.127026 92.284406) (size 0.6) (drill 0.3) (layers "F.Cu" "B.Cu") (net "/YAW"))
 (segment (start 157.087388 97.105428) (end 154.933351 97.105428) (width 0.2) (layer "B.Cu") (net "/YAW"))
 (segment (start 157.928722 96.264094) (end 157.087388 97.105428) (width 0.2) (layer "B.Cu") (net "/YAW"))
 (segment (start 160.127026 92.284406) (end 157.928722 94.48271) (width 0.2) (layer "B.Cu") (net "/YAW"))
 (segment (start 157.928722 94.48271) (end 157.928722 96.264094) (width 0.2) (layer "B.Cu") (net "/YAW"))
 (segment (start 136.933351 92.125921) (end 143.443612 85.61566) (width 0.2) (layer "F.Cu") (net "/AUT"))
 (segment (start 143.443612 85.61566) (end 148.817216 85.61566) (width 0.2) (layer "F.Cu") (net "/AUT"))
 (segment (start 148.817216 85.61566) (end 148.84108 85.61566) (width 0.2) (layer "F.Cu") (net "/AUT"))
 (via (at 148.817216 85.61566) (size 0.6) (drill 0.3) (layers "F.Cu" "B.Cu") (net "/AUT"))
 (segment (start 198.220469 81.920469) (end 201 84.7) (width 0.2) (layer "B.Cu") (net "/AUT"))
 (segment (start 152.512407 81.920469) (end 198.220469 81.920469) (width 0.2) (layer "B.Cu") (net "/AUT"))
 (segment (start 148.817216 85.61566) (end 152.512407 81.920469) (width 0.2) (layer "B.Cu") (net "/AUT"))
 (segment (start 162.825718 100.851937) (end 162.774715 100.90294) (width 0.4) (layer "F.Cu") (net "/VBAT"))
 (segment (start 158.478331 96.438795) (end 160.066447 98.026911) (width 0.4) (layer "F.Cu") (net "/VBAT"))
 (segment (start 124.117811 101.10003) (end 127.796944 101.10003) (width 0.4) (layer "F.Cu") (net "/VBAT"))
 (segment (start 160.066447 98.026911) (end 162.825718 98.026911) (width 0.4) (layer "F.Cu") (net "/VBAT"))
 (segment (start 162.825718 98.026911) (end 162.825718 100.851937) (width 0.4) (layer "F.Cu") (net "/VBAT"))
 (segment (start 154.933351 86.945428) (end 158.478331 90.490408) (width 0.4) (layer "F.Cu") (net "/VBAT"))
 (segment (start 127.796944 101.10003) (end 127.866096 101.030878) (width 0.4) (layer "F.Cu") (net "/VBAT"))
 (segment (start 158.478331 90.490408) (end 158.478331 96.438795) (width 0.4) (layer "F.Cu") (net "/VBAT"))
 (via (at 124.117811 101.10003) (size 0.6) (drill 0.3) (layers "F.Cu" "B.Cu") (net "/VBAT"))
 (segment (start 147.296472 86.945428) (end 139.695447 79.344403) (width 0.4) (layer "B.Cu") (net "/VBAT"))
 (segment (start 123.814597 100.796816) (end 124.117811 101.10003) (width 0.4) (layer "B.Cu") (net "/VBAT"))
 (segment (start 154.933351 86.945428) (end 147.296472 86.945428) (width 0.4) (layer "B.Cu") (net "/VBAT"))
 (segment (start 139.695447 79.344403) (end 123.814597 79.344403) (width 0.4) (layer "B.Cu") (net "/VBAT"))
 (segment (start 123.814597 79.344403) (end 123.814597 100.796816) (width 0.4) (layer "B.Cu") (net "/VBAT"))
 (segment (start 158.839543 115.360681) (end 162.387856 115.360681) (width 0.2) (layer "F.Cu") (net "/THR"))
 (segment (start 154.933351 109.805428) (end 154.933351 114.905906) (width 0.2) (layer "F.Cu") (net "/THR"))
 (segment (start 155.787272 115.759827) (end 158.440397 115.759827) (width 0.2) (layer "F.Cu") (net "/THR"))
 (segment (start 158.440397 115.759827) (end 158.839543 115.360681) (width 0.2) (layer "F.Cu") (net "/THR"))
 (segment (start 154.933351 114.905906) (end 155.787272 115.759827) (width 0.2) (layer "F.Cu") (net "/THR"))
 (segment (start 132.143412 86.81285) (end 132.205575 86.750687) (width 0.2) (layer "F.Cu") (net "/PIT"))
 (segment (start 132.205575 86.750687) (end 132.736902 87.282014) (width 0.2) (layer "F.Cu") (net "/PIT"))
 (segment (start 128.356566 86.81285) (end 132.143412 86.81285) (width 0.2) (layer "F.Cu") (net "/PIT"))
 (segment (start 132.736902 95.42388) (end 132.736902 95.468801) (width 0.2) (layer "F.Cu") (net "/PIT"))
 (segment (start 132.205575 86.750687) (end 132.206277 86.749985) (width 0.2) (layer "F.Cu") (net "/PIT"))
 (segment (start 132.736902 87.282014) (end 132.736902 95.42388) (width 0.2) (layer "F.Cu") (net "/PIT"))
 (via (at 132.736902 95.42388) (size 0.6) (drill 0.3) (layers "F.Cu" "B.Cu") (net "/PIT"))
 (segment (start 132.736902 95.42388) (end 132.736902 98.089472) (width 0.2) (layer "B.Cu") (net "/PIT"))
 (segment (start 132.736902 98.089472) (end 136.933351 102.285921) (width 0.2) (layer "B.Cu") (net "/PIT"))
 (segment (start 136.410002 81.163679) (end 136.945984 81.699661) (width 0.2) (layer "F.Cu") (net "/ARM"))
 (segment (start 114.957992 81.163679) (end 136.410002 81.163679) (width 0.2) (layer "F.Cu") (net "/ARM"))
 (via (at 136.945984 81.699661) (size 0.6) (drill 0.3) (layers "F.Cu" "B.Cu") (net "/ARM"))
 (segment (start 136.933351 81.712294) (end 136.933351 87.045921) (width 0.2) (layer "B.Cu") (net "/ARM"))
 (segment (start 136.945984 81.699661) (end 136.933351 81.712294) (width 0.2) (layer "B.Cu") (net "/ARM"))
 (segment (start 139.836522 81.931108) (end 137.769093 79.863679) (width 0.2) (layer "F.Cu") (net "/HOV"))
 (segment (start 98.386321 79.863679) (end 95.25 83) (width 0.2) (layer "F.Cu") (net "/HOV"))
 (segment (start 137.769093 79.863679) (end 98.386321 79.863679) (width 0.2) (layer "F.Cu") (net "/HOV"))
 (via (at 139.836522 81.931108) (size 0.6) (drill 0.3) (layers "F.Cu" "B.Cu") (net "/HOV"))
 (segment (start 136.933351 89.585921) (end 139.836522 86.68275) (width 0.2) (layer "B.Cu") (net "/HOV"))
 (segment (start 139.836522 86.68275) (end 139.836522 81.931108) (width 0.2) (layer "B.Cu") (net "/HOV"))
 (segment (start 139.836522 81.931108) (end 139.836522 81.908648) (width 0.2) (layer "B.Cu") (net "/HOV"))
 (segment (start 139.984142 107.876712) (end 136.933351 104.825921) (width 0.2) (layer "F.Cu") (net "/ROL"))
 (segment (start 138.743584 112.056428) (end 139.984142 110.81587) (width 0.2) (layer "F.Cu") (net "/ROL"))
 (segment (start 127.871225 112.056428) (end 138.743584 112.056428) (width 0.2) (layer "F.Cu") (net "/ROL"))
 (segment (start 139.984142 110.81587) (end 139.984142 107.876712) (width 0.2) (layer "F.Cu") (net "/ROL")))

